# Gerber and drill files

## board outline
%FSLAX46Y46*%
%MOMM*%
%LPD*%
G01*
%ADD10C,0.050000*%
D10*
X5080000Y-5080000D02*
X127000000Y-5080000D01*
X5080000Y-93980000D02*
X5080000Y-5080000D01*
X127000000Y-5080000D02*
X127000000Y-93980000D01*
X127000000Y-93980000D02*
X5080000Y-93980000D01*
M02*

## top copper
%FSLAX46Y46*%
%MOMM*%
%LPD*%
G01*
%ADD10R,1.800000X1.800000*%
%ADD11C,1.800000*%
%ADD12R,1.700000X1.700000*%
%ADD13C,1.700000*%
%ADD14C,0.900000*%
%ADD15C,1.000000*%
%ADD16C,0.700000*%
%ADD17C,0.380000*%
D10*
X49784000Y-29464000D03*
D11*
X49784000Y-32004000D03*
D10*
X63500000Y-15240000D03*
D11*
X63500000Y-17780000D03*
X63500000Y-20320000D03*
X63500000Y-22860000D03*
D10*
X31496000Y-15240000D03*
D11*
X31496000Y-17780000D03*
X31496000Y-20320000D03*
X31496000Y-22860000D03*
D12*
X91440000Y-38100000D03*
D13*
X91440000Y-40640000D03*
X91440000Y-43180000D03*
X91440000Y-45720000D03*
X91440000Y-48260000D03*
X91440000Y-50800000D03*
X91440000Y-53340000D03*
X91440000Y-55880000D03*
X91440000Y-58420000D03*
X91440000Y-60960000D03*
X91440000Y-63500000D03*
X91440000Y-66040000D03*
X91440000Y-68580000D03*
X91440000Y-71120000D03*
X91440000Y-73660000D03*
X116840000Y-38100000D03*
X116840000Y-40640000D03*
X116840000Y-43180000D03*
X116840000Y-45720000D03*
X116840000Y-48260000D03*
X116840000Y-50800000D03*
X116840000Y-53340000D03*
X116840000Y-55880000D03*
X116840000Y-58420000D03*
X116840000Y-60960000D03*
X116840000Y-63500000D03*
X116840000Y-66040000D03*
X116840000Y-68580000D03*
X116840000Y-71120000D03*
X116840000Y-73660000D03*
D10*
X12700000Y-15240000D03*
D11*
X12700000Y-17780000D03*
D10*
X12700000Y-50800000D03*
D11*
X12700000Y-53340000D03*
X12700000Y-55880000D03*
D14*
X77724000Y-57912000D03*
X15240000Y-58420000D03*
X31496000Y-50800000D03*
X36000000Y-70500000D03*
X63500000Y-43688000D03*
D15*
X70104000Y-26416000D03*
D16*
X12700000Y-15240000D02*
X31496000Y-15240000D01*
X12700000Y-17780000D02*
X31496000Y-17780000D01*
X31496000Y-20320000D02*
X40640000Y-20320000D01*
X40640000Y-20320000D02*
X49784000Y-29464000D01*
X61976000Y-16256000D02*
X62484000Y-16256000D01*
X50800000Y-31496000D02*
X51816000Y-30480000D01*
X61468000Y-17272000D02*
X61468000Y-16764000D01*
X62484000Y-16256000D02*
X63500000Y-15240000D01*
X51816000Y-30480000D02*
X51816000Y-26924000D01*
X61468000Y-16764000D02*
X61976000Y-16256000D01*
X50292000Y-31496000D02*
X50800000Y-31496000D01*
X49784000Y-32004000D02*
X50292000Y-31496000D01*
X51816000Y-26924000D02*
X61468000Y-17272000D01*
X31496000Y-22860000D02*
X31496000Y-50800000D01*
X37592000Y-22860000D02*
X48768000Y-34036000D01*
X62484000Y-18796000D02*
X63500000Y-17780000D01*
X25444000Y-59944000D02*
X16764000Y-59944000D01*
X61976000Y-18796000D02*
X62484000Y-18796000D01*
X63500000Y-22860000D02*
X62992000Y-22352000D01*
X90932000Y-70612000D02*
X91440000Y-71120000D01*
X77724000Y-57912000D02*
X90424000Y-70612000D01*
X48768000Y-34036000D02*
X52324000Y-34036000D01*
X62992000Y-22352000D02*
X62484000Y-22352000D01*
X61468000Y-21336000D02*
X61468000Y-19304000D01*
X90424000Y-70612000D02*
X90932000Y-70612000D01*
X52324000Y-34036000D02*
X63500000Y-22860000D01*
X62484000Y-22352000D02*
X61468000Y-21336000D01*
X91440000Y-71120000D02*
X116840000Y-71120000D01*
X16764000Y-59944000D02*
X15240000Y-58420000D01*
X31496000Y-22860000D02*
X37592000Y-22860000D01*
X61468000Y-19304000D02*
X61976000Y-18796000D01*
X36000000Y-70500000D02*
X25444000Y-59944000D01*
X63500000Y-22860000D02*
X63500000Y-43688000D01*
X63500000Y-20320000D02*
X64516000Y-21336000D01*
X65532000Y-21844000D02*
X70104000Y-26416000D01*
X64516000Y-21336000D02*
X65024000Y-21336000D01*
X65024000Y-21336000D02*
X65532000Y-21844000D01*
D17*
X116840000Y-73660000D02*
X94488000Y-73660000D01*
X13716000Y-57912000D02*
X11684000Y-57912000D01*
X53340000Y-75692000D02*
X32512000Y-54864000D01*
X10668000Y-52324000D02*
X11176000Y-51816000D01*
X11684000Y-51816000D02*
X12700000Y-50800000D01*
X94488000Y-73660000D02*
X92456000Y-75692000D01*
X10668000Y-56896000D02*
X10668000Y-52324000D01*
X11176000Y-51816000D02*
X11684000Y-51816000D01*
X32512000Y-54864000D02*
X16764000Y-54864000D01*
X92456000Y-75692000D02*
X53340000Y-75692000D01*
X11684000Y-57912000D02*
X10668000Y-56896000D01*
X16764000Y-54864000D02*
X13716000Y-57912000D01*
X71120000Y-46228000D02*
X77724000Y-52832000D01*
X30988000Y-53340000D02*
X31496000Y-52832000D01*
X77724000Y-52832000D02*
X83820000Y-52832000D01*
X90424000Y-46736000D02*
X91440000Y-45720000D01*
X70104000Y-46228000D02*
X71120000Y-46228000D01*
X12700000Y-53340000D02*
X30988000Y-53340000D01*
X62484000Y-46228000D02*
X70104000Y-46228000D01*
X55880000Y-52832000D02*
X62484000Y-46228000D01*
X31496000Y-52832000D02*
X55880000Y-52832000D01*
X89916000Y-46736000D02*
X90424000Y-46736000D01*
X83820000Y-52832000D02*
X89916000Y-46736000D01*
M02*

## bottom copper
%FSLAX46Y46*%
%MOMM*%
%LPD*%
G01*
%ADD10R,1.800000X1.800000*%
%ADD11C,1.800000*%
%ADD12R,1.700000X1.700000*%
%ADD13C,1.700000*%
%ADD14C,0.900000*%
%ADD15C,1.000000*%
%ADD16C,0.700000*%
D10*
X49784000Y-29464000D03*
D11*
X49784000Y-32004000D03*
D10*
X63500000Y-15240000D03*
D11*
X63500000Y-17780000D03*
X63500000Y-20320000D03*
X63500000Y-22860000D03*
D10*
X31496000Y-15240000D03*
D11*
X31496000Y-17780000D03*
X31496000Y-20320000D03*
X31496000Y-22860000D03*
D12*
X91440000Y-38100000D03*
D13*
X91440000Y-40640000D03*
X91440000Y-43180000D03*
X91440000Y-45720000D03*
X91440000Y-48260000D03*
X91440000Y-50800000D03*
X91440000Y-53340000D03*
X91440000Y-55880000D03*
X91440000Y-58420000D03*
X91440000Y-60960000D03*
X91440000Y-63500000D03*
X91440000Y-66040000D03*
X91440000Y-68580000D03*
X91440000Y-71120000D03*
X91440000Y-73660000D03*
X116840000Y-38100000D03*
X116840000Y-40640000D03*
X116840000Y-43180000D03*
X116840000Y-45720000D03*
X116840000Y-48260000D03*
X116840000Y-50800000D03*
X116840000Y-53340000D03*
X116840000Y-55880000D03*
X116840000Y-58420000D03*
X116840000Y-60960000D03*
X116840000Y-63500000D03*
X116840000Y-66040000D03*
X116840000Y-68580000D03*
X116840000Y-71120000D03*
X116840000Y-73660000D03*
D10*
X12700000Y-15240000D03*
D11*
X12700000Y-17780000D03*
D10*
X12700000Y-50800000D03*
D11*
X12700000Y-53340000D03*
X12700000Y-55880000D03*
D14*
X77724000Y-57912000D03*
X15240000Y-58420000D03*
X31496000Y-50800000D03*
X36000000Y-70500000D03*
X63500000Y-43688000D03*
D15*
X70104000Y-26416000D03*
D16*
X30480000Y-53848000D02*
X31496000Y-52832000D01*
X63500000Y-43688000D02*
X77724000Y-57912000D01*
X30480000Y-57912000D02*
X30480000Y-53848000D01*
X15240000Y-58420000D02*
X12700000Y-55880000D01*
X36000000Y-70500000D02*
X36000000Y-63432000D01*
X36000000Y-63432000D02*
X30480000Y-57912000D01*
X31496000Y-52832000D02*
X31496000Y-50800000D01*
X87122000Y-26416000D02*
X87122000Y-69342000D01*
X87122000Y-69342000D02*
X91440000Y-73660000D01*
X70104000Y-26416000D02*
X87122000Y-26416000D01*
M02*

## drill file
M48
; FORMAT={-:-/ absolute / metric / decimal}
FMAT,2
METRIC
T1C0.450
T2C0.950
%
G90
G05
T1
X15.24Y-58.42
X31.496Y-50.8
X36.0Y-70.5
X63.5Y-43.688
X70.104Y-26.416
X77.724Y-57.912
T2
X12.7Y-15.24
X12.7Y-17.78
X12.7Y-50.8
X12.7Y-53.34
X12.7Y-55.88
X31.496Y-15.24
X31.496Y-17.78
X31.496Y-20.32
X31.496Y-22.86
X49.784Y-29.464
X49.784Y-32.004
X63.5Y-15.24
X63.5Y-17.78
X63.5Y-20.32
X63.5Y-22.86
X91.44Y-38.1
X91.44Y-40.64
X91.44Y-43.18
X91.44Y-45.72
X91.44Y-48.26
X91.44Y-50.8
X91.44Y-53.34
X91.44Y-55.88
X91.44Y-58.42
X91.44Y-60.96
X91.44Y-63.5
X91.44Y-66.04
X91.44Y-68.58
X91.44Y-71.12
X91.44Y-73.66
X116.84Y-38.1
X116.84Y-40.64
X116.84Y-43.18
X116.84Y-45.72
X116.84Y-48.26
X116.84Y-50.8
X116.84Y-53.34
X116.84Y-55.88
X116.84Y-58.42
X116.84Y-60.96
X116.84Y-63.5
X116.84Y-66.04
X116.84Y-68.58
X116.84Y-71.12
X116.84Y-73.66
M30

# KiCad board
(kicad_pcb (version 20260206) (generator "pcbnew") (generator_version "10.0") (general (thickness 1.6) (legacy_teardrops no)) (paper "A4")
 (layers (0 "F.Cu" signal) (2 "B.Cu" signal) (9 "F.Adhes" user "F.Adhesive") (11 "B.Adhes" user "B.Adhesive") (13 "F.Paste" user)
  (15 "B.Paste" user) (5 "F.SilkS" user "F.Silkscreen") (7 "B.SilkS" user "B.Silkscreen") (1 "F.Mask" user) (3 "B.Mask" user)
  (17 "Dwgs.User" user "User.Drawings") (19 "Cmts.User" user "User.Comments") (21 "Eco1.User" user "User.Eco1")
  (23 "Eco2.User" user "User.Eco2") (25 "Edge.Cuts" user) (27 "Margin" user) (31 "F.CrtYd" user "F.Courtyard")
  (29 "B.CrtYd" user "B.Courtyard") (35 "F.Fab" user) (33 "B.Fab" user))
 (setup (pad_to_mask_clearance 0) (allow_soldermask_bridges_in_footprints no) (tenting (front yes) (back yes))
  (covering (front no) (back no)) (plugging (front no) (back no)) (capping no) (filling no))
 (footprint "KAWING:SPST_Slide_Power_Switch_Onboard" (layer "F.Cu") (at 49.784 29.464)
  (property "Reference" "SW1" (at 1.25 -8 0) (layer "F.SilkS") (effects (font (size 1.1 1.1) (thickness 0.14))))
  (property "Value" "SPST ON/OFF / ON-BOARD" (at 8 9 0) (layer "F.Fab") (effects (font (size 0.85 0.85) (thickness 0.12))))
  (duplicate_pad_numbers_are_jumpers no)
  (pad "1" thru_hole rect (at 0 0) (size 1.8 1.8) (drill 0.95) (layers "*.Cu" "*.Mask") (remove_unused_layers no) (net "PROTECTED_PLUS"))
  (pad "2" thru_hole circle (at 0 2.54) (size 1.8 1.8) (drill 0.95) (layers "*.Cu" "*.Mask") (remove_unused_layers no)
   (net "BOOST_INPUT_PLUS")))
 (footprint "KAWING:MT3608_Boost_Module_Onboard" (layer "F.Cu") (at 63.5 15.24)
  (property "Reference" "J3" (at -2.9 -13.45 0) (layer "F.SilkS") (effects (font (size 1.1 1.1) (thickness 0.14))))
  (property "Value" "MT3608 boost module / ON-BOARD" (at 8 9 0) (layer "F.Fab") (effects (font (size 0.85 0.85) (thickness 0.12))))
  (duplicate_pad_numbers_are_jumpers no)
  (pad "1" thru_hole rect (at 0 0) (size 1.8 1.8) (drill 0.95) (layers "*.Cu" "*.Mask") (remove_unused_layers no) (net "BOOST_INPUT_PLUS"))
  (pad "2" thru_hole circle (at 0 2.54) (size 1.8 1.8) (drill 0.95) (layers "*.Cu" "*.Mask") (remove_unused_layers no) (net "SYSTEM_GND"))
  (pad "3" thru_hole circle (at 0 5.08) (size 1.8 1.8) (drill 0.95) (layers "*.Cu" "*.Mask") (remove_unused_layers no) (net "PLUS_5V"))
  (pad "4" thru_hole circle (at 0 7.62) (size 1.8 1.8) (drill 0.95) (layers "*.Cu" "*.Mask") (remove_unused_layers no) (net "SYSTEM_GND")))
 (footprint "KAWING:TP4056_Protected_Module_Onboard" (layer "F.Cu") (at 31.496 15.24)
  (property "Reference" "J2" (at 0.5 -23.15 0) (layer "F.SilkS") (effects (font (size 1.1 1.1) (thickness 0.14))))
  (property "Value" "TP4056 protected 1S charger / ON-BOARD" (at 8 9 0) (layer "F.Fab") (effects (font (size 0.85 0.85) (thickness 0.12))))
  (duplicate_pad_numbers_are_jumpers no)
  (pad "1" thru_hole rect (at 0 0) (size 1.8 1.8) (drill 0.95) (layers "*.Cu" "*.Mask") (remove_unused_layers no) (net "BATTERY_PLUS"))
  (pad "2" thru_hole circle (at 0 2.54) (size 1.8 1.8) (drill 0.95) (layers "*.Cu" "*.Mask") (remove_unused_layers no) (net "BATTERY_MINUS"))
  (pad "3" thru_hole circle (at 0 5.08) (size 1.8 1.8) (drill 0.95) (layers "*.Cu" "*.Mask") (remove_unused_layers no)
   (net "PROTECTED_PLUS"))
  (pad "4" thru_hole circle (at 0 7.62) (size 1.8 1.8) (drill 0.95) (layers "*.Cu" "*.Mask") (remove_unused_layers no) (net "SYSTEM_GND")))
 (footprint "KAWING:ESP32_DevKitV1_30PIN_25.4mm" (layer "F.Cu") (at 91.44 38.1)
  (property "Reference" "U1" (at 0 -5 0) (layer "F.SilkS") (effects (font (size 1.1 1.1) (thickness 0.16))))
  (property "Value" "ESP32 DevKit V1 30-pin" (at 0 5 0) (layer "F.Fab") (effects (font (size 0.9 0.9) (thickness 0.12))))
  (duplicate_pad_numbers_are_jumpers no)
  (pad "1" thru_hole rect (at 0 0) (size 1.7 1.7) (drill 0.95) (layers "*.Cu" "*.Mask") (remove_unused_layers no))
  (pad "2" thru_hole circle (at 0 2.54) (size 1.7 1.7) (drill 0.95) (layers "*.Cu" "*.Mask") (remove_unused_layers no))
  (pad "3" thru_hole circle (at 0 5.08) (size 1.7 1.7) (drill 0.95) (layers "*.Cu" "*.Mask") (remove_unused_layers no))
  (pad "4" thru_hole circle (at 0 7.62) (size 1.7 1.7) (drill 0.95) (layers "*.Cu" "*.Mask") (remove_unused_layers no) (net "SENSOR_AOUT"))
  (pad "5" thru_hole circle (at 0 10.16) (size 1.7 1.7) (drill 0.95) (layers "*.Cu" "*.Mask") (remove_unused_layers no))
  (pad "6" thru_hole circle (at 0 12.7) (size 1.7 1.7) (drill 0.95) (layers "*.Cu" "*.Mask") (remove_unused_layers no))
  (pad "7" thru_hole circle (at 0 15.24) (size 1.7 1.7) (drill 0.95) (layers "*.Cu" "*.Mask") (remove_unused_layers no))
  (pad "8" thru_hole circle (at 0 17.78) (size 1.7 1.7) (drill 0.95) (layers "*.Cu" "*.Mask") (remove_unused_layers no))
  (pad "9" thru_hole circle (at 0 20.32) (size 1.7 1.7) (drill 0.95) (layers "*.Cu" "*.Mask") (remove_unused_layers no))
  (pad "10" thru_hole circle (at 0 22.86) (size 1.7 1.7) (drill 0.95) (layers "*.Cu" "*.Mask") (remove_unused_layers no))
  (pad "11" thru_hole circle (at 0 25.4) (size 1.7 1.7) (drill 0.95) (layers "*.Cu" "*.Mask") (remove_unused_layers no))
  (pad "12" thru_hole circle (at 0 27.94) (size 1.7 1.7) (drill 0.95) (layers "*.Cu" "*.Mask") (remove_unused_layers no))
  (pad "13" thru_hole circle (at 0 30.48) (size 1.7 1.7) (drill 0.95) (layers "*.Cu" "*.Mask") (remove_unused_layers no))
  (pad "14" thru_hole circle (at 0 33.02) (size 1.7 1.7) (drill 0.95) (layers "*.Cu" "*.Mask") (remove_unused_layers no) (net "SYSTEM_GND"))
  (pad "15" thru_hole circle (at 0 35.56) (size 1.7 1.7) (drill 0.95) (layers "*.Cu" "*.Mask") (remove_unused_layers no) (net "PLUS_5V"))
  (pad "16" thru_hole circle (at 25.4 0) (size 1.7 1.7) (drill 0.95) (layers "*.Cu" "*.Mask") (remove_unused_layers no))
  (pad "17" thru_hole circle (at 25.4 2.54) (size 1.7 1.7) (drill 0.95) (layers "*.Cu" "*.Mask") (remove_unused_layers no))
  (pad "18" thru_hole circle (at 25.4 5.08) (size 1.7 1.7) (drill 0.95) (layers "*.Cu" "*.Mask") (remove_unused_layers no))
  (pad "19" thru_hole circle (at 25.4 7.62) (size 1.7 1.7) (drill 0.95) (layers "*.Cu" "*.Mask") (remove_unused_layers no))
  (pad "20" thru_hole circle (at 25.4 10.16) (size 1.7 1.7) (drill 0.95) (layers "*.Cu" "*.Mask") (remove_unused_layers no))
  (pad "21" thru_hole circle (at 25.4 12.7) (size 1.7 1.7) (drill 0.95) (layers "*.Cu" "*.Mask") (remove_unused_layers no))
  (pad "22" thru_hole circle (at 25.4 15.24) (size 1.7 1.7) (drill 0.95) (layers "*.Cu" "*.Mask") (remove_unused_layers no))
  (pad "23" thru_hole circle (at 25.4 17.78) (size 1.7 1.7) (drill 0.95) (layers "*.Cu" "*.Mask") (remove_unused_layers no))
  (pad "24" thru_hole circle (at 25.4 20.32) (size 1.7 1.7) (drill 0.95) (layers "*.Cu" "*.Mask") (remove_unused_layers no))
  (pad "25" thru_hole circle (at 25.4 22.86) (size 1.7 1.7) (drill 0.95) (layers "*.Cu" "*.Mask") (remove_unused_layers no))
  (pad "26" thru_hole circle (at 25.4 25.4) (size 1.7 1.7) (drill 0.95) (layers "*.Cu" "*.Mask") (remove_unused_layers no))
  (pad "27" thru_hole circle (at 25.4 27.94) (size 1.7 1.7) (drill 0.95) (layers "*.Cu" "*.Mask") (remove_unused_layers no))
  (pad "28" thru_hole circle (at 25.4 30.48) (size 1.7 1.7) (drill 0.95) (layers "*.Cu" "*.Mask") (remove_unused_layers no))
  (pad "29" thru_hole circle (at 25.4 33.02) (size 1.7 1.7) (drill 0.95) (layers "*.Cu" "*.Mask") (remove_unused_layers no)
   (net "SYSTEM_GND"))
  (pad "30" thru_hole circle (at 25.4 35.56) (size 1.7 1.7) (drill 0.95) (layers "*.Cu" "*.Mask") (remove_unused_layers no)
   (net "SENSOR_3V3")))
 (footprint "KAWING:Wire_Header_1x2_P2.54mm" (layer "F.Cu") (at 12.7 15.24)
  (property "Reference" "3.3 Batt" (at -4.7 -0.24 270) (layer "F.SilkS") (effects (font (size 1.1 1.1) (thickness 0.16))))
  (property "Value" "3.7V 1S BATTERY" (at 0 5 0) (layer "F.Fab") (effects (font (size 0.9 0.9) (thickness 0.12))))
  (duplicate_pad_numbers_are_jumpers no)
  (pad "1" thru_hole rect (at 0 0) (size 1.8 1.8) (drill 0.95) (layers "*.Cu" "*.Mask") (remove_unused_layers no) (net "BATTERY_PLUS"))
  (pad "2" thru_hole circle (at 0 2.54) (size 1.8 1.8) (drill 0.95) (layers "*.Cu" "*.Mask") (remove_unused_layers no) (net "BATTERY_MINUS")))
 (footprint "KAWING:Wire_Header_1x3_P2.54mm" (layer "F.Cu") (at 12.7 50.8)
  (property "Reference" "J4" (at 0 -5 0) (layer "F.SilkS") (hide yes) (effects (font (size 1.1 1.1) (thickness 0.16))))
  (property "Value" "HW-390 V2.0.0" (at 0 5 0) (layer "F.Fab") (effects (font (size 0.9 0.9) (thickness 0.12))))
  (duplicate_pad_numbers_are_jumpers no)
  (pad "1" thru_hole rect (at 0 0) (size 1.8 1.8) (drill 0.95) (layers "*.Cu" "*.Mask") (remove_unused_layers no) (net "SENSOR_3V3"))
  (pad "2" thru_hole circle (at 0 2.54) (size 1.8 1.8) (drill 0.95) (layers "*.Cu" "*.Mask") (remove_unused_layers no) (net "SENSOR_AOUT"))
  (pad "3" thru_hole circle (at 0 5.08) (size 1.8 1.8) (drill 0.95) (layers "*.Cu" "*.Mask") (remove_unused_layers no) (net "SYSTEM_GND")))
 (gr_line (start 5.08 5.08) (end 127 5.08) (stroke (width 0.05) (type default)) (layer "Edge.Cuts"))
 (gr_line (start 5.08 93.98) (end 5.08 5.08) (stroke (width 0.05) (type default)) (layer "Edge.Cuts"))
 (gr_line (start 127 5.08) (end 127 93.98) (stroke (width 0.05) (type default)) (layer "Edge.Cuts"))
 (gr_line (start 127 93.98) (end 5.08 93.98) (stroke (width 0.05) (type default)) (layer "Edge.Cuts"))
 (segment (start 12.7 15.24) (end 31.496 15.24) (width 0.7) (layer "F.Cu") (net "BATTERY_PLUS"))
 (segment (start 12.7 17.78) (end 31.496 17.78) (width 0.7) (layer "F.Cu") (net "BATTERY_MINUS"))
 (segment (start 31.496 20.32) (end 40.64 20.32) (width 0.7) (layer "F.Cu") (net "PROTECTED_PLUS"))
 (segment (start 40.64 20.32) (end 49.784 29.464) (width 0.7) (layer "F.Cu") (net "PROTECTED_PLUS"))
 (segment (start 61.976 16.256) (end 62.484 16.256) (width 0.7) (layer "F.Cu") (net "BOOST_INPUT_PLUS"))
 (segment (start 50.8 31.496) (end 51.816 30.48) (width 0.7) (layer "F.Cu") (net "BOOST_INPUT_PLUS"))
 (segment (start 61.468 17.272) (end 61.468 16.764) (width 0.7) (layer "F.Cu") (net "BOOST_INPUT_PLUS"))
 (segment (start 62.484 16.256) (end 63.5 15.24) (width 0.7) (layer "F.Cu") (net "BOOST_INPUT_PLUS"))
 (segment (start 51.816 30.48) (end 51.816 26.924) (width 0.7) (layer "F.Cu") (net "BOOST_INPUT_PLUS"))
 (segment (start 61.468 16.764) (end 61.976 16.256) (width 0.7) (layer "F.Cu") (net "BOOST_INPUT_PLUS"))
 (segment (start 50.292 31.496) (end 50.8 31.496) (width 0.7) (layer "F.Cu") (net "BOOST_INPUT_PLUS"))
 (segment (start 49.784 32.004) (end 50.292 31.496) (width 0.7) (layer "F.Cu") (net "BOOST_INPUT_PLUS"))
 (segment (start 51.816 26.924) (end 61.468 17.272) (width 0.7) (layer "F.Cu") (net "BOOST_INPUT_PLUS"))
 (segment (start 31.496 22.86) (end 31.496 50.8) (width 0.7) (layer "F.Cu") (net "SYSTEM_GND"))
 (segment (start 37.592 22.86) (end 48.768 34.036) (width 0.7) (layer "F.Cu") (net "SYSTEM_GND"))
 (segment (start 62.484 18.796) (end 63.5 17.78) (width 0.7) (layer "F.Cu") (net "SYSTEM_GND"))
 (segment (start 25.444 59.944) (end 16.764 59.944) (width 0.7) (layer "F.Cu") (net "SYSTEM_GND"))
 (segment (start 61.976 18.796) (end 62.484 18.796) (width 0.7) (layer "F.Cu") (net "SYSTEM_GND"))
 (segment (start 63.5 22.86) (end 62.992 22.352) (width 0.7) (layer "F.Cu") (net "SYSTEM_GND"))
 (segment (start 90.932 70.612) (end 91.44 71.12) (width 0.7) (layer "F.Cu") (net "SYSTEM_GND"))
 (segment (start 77.724 57.912) (end 90.424 70.612) (width 0.7) (layer "F.Cu") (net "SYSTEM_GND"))
 (segment (start 48.768 34.036) (end 52.324 34.036) (width 0.7) (layer "F.Cu") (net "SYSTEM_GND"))
 (segment (start 62.992 22.352) (end 62.484 22.352) (width 0.7) (layer "F.Cu") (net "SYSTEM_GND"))
 (segment (start 61.468 21.336) (end 61.468 19.304) (width 0.7) (layer "F.Cu") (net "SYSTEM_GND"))
 (segment (start 90.424 70.612) (end 90.932 70.612) (width 0.7) (layer "F.Cu") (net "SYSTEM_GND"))
 (segment (start 52.324 34.036) (end 63.5 22.86) (width 0.7) (layer "F.Cu") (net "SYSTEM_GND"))
 (segment (start 62.484 22.352) (end 61.468 21.336) (width 0.7) (layer "F.Cu") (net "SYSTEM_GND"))
 (segment (start 91.44 71.12) (end 116.84 71.12) (width 0.7) (layer "F.Cu") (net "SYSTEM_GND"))
 (segment (start 16.764 59.944) (end 15.24 58.42) (width 0.7) (layer "F.Cu") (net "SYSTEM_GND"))
 (segment (start 31.496 22.86) (end 37.592 22.86) (width 0.7) (layer "F.Cu") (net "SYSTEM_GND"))
 (segment (start 61.468 19.304) (end 61.976 18.796) (width 0.7) (layer "F.Cu") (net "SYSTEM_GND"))
 (segment (start 36 70.5) (end 25.444 59.944) (width 0.7) (layer "F.Cu") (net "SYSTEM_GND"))
 (segment (start 63.5 22.86) (end 63.5 43.688) (width 0.7) (layer "F.Cu") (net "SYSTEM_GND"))
 (via (at 77.724 57.912) (size 0.9) (drill 0.45) (layers "F.Cu" "B.Cu") (capping no) (covering (front no) (back no))
  (plugging (front no) (back no)) (filling no) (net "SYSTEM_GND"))
 (via (at 15.24 58.42) (size 0.9) (drill 0.45) (layers "F.Cu" "B.Cu") (capping no) (covering (front no) (back no))
  (plugging (front no) (back no)) (filling no) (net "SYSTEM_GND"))
 (via (at 31.496 50.8) (size 0.9) (drill 0.45) (layers "F.Cu" "B.Cu") (capping no) (covering (front no) (back no))
  (plugging (front no) (back no)) (filling no) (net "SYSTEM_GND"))
 (via (at 36 70.5) (size 0.9) (drill 0.45) (layers "F.Cu" "B.Cu") (capping no) (covering (front no) (back no))
  (plugging (front no) (back no)) (filling no) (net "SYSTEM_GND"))
 (via (at 63.5 43.688) (size 0.9) (drill 0.45) (layers "F.Cu" "B.Cu") (capping no) (covering (front no) (back no))
  (plugging (front no) (back no)) (filling no) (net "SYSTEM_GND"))
 (segment (start 30.48 53.848) (end 31.496 52.832) (width 0.7) (layer "B.Cu") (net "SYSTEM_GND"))
 (segment (start 63.5 43.688) (end 77.724 57.912) (width 0.7) (layer "B.Cu") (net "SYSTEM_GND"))
 (segment (start 30.48 57.912) (end 30.48 53.848) (width 0.7) (layer "B.Cu") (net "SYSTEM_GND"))
 (segment (start 15.24 58.42) (end 12.7 55.88) (width 0.7) (layer "B.Cu") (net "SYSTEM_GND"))
 (segment (start 36 70.5) (end 36 63.432) (width 0.7) (layer "B.Cu") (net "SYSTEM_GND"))
 (segment (start 36 63.432) (end 30.48 57.912) (width 0.7) (layer "B.Cu") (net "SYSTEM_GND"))
 (segment (start 31.496 52.832) (end 31.496 50.8) (width 0.7) (layer "B.Cu") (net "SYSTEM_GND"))
 (segment (start 63.5 20.32) (end 64.516 21.336) (width 0.7) (layer "F.Cu") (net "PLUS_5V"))
 (segment (start 65.532 21.844) (end 70.104 26.416) (width 0.7) (layer "F.Cu") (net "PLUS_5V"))
 (segment (start 64.516 21.336) (end 65.024 21.336) (width 0.7) (layer "F.Cu") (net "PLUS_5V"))
 (segment (start 65.024 21.336) (end 65.532 21.844) (width 0.7) (layer "F.Cu") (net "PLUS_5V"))
 (via (at 70.104 26.416) (size 1) (drill 0.45) (layers "F.Cu" "B.Cu") (capping no) (covering (front no) (back no))
  (plugging (front no) (back no)) (filling no) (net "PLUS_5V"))
 (segment (start 87.122 26.416) (end 87.122 69.342) (width 0.7) (layer "B.Cu") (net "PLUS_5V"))
 (segment (start 87.122 69.342) (end 91.44 73.66) (width 0.7) (layer "B.Cu") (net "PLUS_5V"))
 (segment (start 70.104 26.416) (end 87.122 26.416) (width 0.7) (layer "B.Cu") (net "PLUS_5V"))
 (segment (start 116.84 73.66) (end 94.488 73.66) (width 0.38) (layer "F.Cu") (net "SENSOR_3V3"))
 (segment (start 13.716 57.912) (end 11.684 57.912) (width 0.38) (layer "F.Cu") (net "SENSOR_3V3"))
 (segment (start 53.34 75.692) (end 32.512 54.864) (width 0.38) (layer "F.Cu") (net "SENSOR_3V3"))
 (segment (start 10.668 52.324) (end 11.176 51.816) (width 0.38) (layer "F.Cu") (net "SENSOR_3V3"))
 (segment (start 11.684 51.816) (end 12.7 50.8) (width 0.38) (layer "F.Cu") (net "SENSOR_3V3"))
 (segment (start 94.488 73.66) (end 92.456 75.692) (width 0.38) (layer "F.Cu") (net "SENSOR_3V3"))
 (segment (start 10.668 56.896) (end 10.668 52.324) (width 0.38) (layer "F.Cu") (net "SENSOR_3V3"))
 (segment (start 11.176 51.816) (end 11.684 51.816) (width 0.38) (layer "F.Cu") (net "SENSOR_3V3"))
 (segment (start 32.512 54.864) (end 16.764 54.864) (width 0.38) (layer "F.Cu") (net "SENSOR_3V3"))
 (segment (start 92.456 75.692) (end 53.34 75.692) (width 0.38) (layer "F.Cu") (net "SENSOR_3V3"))
 (segment (start 11.684 57.912) (end 10.668 56.896) (width 0.38) (layer "F.Cu") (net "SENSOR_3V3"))
 (segment (start 16.764 54.864) (end 13.716 57.912) (width 0.38) (layer "F.Cu") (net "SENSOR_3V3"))
 (segment (start 71.12 46.228) (end 77.724 52.832) (width 0.38) (layer "F.Cu") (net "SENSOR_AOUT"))
 (segment (start 30.988 53.34) (end 31.496 52.832) (width 0.38) (layer "F.Cu") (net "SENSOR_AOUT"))
 (segment (start 77.724 52.832) (end 83.82 52.832) (width 0.38) (layer "F.Cu") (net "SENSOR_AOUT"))
 (segment (start 90.424 46.736) (end 91.44 45.72) (width 0.38) (layer "F.Cu") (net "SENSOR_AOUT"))
 (segment (start 70.104 46.228) (end 71.12 46.228) (width 0.38) (layer "F.Cu") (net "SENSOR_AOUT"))
 (segment (start 12.7 53.34) (end 30.988 53.34) (width 0.38) (layer "F.Cu") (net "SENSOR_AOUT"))
 (segment (start 62.484 46.228) (end 70.104 46.228) (width 0.38) (layer "F.Cu") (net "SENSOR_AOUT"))
 (segment (start 55.88 52.832) (end 62.484 46.228) (width 0.38) (layer "F.Cu") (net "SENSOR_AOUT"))
 (segment (start 31.496 52.832) (end 55.88 52.832) (width 0.38) (layer "F.Cu") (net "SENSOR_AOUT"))
 (segment (start 89.916 46.736) (end 90.424 46.736) (width 0.38) (layer "F.Cu") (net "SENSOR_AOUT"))
 (segment (start 83.82 52.832) (end 89.916 46.736) (width 0.38) (layer "F.Cu") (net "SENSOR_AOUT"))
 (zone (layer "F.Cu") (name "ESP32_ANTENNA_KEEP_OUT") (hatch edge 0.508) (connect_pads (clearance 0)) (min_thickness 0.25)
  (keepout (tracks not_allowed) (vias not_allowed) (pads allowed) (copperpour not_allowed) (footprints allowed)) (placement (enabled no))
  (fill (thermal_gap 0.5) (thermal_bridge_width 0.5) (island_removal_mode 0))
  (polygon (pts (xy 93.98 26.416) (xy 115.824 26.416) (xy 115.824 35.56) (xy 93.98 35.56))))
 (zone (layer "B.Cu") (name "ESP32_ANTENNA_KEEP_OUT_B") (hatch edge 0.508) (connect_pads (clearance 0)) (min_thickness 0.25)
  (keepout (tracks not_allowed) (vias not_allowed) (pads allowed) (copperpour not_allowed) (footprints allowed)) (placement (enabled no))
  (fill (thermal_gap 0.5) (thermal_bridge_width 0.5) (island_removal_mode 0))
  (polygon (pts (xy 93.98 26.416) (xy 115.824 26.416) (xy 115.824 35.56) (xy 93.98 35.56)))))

